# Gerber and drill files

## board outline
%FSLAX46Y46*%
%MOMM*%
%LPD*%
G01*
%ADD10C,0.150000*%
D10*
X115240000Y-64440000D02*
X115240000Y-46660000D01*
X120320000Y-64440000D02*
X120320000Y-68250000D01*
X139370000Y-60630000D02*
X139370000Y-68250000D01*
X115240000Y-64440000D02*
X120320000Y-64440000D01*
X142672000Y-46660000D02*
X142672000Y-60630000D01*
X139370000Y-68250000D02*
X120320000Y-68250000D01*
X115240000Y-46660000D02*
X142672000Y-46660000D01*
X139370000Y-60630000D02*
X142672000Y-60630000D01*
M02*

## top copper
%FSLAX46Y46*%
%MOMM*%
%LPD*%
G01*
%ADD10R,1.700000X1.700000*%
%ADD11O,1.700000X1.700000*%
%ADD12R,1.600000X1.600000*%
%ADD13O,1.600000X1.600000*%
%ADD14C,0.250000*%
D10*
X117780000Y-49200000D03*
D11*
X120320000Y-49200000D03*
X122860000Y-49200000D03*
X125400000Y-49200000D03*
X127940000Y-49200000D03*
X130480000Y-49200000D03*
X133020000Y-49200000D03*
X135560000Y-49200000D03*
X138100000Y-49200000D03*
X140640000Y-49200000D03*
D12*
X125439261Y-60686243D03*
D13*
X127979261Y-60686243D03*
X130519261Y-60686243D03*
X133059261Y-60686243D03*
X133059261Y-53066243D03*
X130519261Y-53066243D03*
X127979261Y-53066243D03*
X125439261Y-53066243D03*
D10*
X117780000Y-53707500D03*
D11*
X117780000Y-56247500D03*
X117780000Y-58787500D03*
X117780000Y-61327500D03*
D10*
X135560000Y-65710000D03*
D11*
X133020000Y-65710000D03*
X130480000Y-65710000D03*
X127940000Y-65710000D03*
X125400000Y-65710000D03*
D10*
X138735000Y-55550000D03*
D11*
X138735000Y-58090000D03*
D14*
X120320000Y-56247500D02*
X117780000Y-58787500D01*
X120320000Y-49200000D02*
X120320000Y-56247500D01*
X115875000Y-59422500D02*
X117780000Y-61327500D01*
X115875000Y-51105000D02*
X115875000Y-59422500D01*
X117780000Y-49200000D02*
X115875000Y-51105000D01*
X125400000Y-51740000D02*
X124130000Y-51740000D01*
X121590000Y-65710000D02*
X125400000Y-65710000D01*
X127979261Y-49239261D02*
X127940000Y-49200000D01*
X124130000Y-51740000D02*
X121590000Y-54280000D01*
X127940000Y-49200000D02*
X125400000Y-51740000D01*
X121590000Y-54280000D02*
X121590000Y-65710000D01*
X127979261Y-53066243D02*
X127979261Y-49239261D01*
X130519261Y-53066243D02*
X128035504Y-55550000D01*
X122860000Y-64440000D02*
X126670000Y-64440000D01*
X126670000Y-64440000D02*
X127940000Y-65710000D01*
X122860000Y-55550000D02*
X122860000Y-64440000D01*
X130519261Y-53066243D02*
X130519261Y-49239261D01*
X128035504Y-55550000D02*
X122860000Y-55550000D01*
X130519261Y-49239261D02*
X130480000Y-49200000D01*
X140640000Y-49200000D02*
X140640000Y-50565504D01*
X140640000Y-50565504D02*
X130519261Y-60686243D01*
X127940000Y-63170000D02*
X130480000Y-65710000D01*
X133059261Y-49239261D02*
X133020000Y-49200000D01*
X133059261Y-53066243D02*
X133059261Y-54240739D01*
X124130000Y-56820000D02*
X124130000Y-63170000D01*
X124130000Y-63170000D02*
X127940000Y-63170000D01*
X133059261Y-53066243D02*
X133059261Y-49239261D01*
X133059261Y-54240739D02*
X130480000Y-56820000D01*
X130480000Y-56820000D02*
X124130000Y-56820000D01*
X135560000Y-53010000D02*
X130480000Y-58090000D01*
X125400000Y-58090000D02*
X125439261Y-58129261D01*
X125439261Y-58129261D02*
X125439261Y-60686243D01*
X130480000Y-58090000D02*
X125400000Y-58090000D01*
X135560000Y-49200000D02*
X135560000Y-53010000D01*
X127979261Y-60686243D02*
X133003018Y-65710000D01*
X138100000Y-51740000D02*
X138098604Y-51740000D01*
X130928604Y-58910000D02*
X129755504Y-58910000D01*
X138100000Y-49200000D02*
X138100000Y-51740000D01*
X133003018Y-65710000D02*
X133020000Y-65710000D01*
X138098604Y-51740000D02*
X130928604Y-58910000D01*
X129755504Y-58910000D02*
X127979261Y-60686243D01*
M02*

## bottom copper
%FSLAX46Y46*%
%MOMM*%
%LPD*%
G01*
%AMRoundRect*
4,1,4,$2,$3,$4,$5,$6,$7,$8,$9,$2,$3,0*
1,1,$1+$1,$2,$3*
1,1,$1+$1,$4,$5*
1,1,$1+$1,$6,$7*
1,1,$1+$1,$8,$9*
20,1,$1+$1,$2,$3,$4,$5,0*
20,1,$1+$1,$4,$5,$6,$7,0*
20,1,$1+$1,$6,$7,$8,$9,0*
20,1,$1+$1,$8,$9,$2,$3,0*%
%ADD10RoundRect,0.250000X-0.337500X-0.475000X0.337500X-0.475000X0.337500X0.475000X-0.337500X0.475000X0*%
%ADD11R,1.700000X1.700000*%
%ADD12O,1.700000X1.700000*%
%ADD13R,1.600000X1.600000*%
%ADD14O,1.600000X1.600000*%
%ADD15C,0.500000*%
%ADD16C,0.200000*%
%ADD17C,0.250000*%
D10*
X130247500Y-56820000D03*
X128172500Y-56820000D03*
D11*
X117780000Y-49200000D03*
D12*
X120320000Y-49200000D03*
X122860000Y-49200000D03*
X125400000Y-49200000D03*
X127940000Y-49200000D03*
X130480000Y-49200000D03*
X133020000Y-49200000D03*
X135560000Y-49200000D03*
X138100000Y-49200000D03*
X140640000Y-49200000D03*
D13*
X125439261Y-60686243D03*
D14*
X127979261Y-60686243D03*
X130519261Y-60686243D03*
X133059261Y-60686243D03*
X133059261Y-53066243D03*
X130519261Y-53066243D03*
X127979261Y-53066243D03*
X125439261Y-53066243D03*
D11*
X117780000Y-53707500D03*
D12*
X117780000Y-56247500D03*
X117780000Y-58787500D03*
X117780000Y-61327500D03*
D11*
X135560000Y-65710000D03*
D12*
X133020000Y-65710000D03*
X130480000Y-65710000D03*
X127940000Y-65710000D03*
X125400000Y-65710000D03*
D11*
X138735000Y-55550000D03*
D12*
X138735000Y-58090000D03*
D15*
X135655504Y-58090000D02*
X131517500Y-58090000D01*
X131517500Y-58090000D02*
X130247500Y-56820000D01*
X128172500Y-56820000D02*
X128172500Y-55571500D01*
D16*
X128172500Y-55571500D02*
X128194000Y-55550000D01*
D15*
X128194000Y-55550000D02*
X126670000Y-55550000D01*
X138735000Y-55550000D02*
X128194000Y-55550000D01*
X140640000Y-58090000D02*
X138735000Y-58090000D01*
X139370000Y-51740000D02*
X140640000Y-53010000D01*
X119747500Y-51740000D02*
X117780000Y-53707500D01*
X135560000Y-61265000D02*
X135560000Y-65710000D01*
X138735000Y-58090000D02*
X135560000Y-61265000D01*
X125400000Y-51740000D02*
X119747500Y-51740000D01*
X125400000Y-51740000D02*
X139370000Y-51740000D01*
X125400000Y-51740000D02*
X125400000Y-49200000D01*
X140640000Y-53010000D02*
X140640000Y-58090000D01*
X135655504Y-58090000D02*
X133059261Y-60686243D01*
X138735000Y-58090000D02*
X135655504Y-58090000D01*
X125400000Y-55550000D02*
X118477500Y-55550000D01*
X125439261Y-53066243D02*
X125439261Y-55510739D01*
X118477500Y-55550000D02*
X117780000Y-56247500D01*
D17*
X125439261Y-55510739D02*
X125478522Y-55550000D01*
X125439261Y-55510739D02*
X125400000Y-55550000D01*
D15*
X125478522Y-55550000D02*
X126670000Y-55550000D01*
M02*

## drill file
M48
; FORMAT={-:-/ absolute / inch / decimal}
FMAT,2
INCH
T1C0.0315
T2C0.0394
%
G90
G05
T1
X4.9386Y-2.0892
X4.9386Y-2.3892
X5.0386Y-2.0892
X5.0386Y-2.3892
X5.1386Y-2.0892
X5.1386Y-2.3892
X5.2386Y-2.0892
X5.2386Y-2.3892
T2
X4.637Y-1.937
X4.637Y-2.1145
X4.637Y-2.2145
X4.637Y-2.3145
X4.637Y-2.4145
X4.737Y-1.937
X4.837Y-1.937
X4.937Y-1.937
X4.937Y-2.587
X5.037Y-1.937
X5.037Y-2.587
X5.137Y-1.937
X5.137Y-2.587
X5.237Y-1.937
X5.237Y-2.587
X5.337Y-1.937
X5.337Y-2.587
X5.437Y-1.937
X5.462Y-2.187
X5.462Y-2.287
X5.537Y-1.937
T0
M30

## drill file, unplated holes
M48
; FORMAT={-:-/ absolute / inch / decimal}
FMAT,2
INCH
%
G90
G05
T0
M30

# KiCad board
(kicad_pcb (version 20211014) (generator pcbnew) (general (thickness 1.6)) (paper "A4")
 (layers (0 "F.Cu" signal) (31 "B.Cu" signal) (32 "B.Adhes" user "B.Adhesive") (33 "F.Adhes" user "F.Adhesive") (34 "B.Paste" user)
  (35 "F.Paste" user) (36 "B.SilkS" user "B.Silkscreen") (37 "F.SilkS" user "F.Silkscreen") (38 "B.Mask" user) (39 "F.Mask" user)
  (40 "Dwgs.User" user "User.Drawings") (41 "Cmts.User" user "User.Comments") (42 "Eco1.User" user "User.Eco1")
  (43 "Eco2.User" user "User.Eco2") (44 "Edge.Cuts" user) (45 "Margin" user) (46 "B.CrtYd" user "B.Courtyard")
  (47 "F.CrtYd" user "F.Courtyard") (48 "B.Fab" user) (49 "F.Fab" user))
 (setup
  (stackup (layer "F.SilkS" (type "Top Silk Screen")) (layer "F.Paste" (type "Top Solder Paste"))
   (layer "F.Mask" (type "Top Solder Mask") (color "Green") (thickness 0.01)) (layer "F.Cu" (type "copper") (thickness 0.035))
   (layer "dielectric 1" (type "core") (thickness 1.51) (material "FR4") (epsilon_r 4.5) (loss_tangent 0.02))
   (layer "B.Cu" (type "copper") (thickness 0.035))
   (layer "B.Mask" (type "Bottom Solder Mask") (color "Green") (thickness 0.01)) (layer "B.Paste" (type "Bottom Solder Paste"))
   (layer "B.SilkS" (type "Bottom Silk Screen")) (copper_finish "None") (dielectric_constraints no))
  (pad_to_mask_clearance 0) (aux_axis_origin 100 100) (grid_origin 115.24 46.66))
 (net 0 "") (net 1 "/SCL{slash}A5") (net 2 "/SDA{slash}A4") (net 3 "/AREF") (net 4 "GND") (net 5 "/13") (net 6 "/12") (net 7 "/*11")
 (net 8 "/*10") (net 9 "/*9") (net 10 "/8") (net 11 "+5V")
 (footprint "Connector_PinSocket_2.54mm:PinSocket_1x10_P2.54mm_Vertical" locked (layer "F.Cu") (at 117.78 49.2 90)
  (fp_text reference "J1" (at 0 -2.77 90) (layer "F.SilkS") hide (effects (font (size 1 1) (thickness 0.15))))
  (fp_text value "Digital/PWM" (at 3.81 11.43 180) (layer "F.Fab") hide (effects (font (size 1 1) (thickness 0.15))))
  (pad "1" thru_hole rect locked (at 0 0 90) (size 1.7 1.7) (drill 1) (layers *.Cu *.Mask) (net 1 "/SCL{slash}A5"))
  (pad "2" thru_hole oval locked (at 0 2.54 90) (size 1.7 1.7) (drill 1) (layers *.Cu *.Mask) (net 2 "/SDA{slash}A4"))
  (pad "3" thru_hole oval locked (at 0 5.08 90) (size 1.7 1.7) (drill 1) (layers *.Cu *.Mask) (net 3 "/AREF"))
  (pad "4" thru_hole oval locked (at 0 7.62 90) (size 1.7 1.7) (drill 1) (layers *.Cu *.Mask) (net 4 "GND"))
  (pad "5" thru_hole oval locked (at 0 10.16 90) (size 1.7 1.7) (drill 1) (layers *.Cu *.Mask) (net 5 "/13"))
  (pad "6" thru_hole oval locked (at 0 12.7 90) (size 1.7 1.7) (drill 1) (layers *.Cu *.Mask) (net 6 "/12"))
  (pad "7" thru_hole oval locked (at 0 15.24 90) (size 1.7 1.7) (drill 1) (layers *.Cu *.Mask) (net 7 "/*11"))
  (pad "8" thru_hole oval locked (at 0 17.78 90) (size 1.7 1.7) (drill 1) (layers *.Cu *.Mask) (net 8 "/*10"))
  (pad "9" thru_hole oval locked (at 0 20.32 90) (size 1.7 1.7) (drill 1) (layers *.Cu *.Mask) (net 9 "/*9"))
  (pad "10" thru_hole oval locked (at 0 22.86 90) (size 1.7 1.7) (drill 1) (layers *.Cu *.Mask) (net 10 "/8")))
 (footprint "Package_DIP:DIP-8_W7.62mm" (layer "F.Cu") (at 125.439261 60.686243 90)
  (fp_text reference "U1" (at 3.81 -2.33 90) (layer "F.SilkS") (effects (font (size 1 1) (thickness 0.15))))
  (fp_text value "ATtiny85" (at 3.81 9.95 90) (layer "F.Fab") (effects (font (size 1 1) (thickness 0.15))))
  (pad "1" thru_hole rect (at 0 0 90) (size 1.6 1.6) (drill 0.8) (layers *.Cu *.Mask) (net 8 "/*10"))
  (pad "2" thru_hole oval (at 0 2.54 90) (size 1.6 1.6) (drill 0.8) (layers *.Cu *.Mask) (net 9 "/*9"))
  (pad "3" thru_hole oval (at 0 5.08 90) (size 1.6 1.6) (drill 0.8) (layers *.Cu *.Mask) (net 10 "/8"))
  (pad "4" thru_hole oval (at 0 7.62 90) (size 1.6 1.6) (drill 0.8) (layers *.Cu *.Mask) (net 4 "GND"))
  (pad "5" thru_hole oval (at 7.62 7.62 90) (size 1.6 1.6) (drill 0.8) (layers *.Cu *.Mask) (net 7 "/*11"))
  (pad "6" thru_hole oval (at 7.62 5.08 90) (size 1.6 1.6) (drill 0.8) (layers *.Cu *.Mask) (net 6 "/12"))
  (pad "7" thru_hole oval (at 7.62 2.54 90) (size 1.6 1.6) (drill 0.8) (layers *.Cu *.Mask) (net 5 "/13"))
  (pad "8" thru_hole oval (at 7.62 0 90) (size 1.6 1.6) (drill 0.8) (layers *.Cu *.Mask) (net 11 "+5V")))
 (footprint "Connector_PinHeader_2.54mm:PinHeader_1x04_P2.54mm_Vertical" (layer "F.Cu") (at 117.78 53.7075)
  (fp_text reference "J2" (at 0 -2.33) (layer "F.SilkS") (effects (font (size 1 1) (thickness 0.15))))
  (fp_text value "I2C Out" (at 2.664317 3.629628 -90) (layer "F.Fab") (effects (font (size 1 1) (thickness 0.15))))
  (pad "1" thru_hole rect (at 0 0) (size 1.7 1.7) (drill 1) (layers *.Cu *.Mask) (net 4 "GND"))
  (pad "2" thru_hole oval (at 0 2.54) (size 1.7 1.7) (drill 1) (layers *.Cu *.Mask) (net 11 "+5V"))
  (pad "3" thru_hole oval (at 0 5.08) (size 1.7 1.7) (drill 1) (layers *.Cu *.Mask) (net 2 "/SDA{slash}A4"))
  (pad "4" thru_hole oval (at 0 7.62) (size 1.7 1.7) (drill 1) (layers *.Cu *.Mask) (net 1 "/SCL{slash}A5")))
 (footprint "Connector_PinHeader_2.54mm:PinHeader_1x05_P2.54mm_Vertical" (layer "F.Cu") (at 135.56 65.71 -90)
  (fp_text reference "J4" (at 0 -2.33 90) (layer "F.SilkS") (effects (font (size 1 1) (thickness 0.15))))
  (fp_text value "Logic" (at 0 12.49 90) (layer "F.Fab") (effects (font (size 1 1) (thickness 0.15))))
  (pad "1" thru_hole rect (at 0 0 270) (size 1.7 1.7) (drill 1) (layers *.Cu *.Mask) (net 4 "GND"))
  (pad "2" thru_hole oval (at 0 2.54 270) (size 1.7 1.7) (drill 1) (layers *.Cu *.Mask) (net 9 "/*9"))
  (pad "3" thru_hole oval (at 0 5.08 270) (size 1.7 1.7) (drill 1) (layers *.Cu *.Mask) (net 7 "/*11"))
  (pad "4" thru_hole oval (at 0 7.62 270) (size 1.7 1.7) (drill 1) (layers *.Cu *.Mask) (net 6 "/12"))
  (pad "5" thru_hole oval (at 0 10.16 270) (size 1.7 1.7) (drill 1) (layers *.Cu *.Mask) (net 5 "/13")))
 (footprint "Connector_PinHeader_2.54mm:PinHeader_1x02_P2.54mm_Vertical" (layer "F.Cu") (at 138.735 55.55)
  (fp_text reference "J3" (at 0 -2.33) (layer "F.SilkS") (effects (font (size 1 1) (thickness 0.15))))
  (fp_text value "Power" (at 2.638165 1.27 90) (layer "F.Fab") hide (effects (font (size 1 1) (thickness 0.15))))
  (pad "1" thru_hole rect (at 0 0) (size 1.7 1.7) (drill 1) (layers *.Cu *.Mask) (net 11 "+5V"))
  (pad "2" thru_hole oval (at 0 2.54) (size 1.7 1.7) (drill 1) (layers *.Cu *.Mask) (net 4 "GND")))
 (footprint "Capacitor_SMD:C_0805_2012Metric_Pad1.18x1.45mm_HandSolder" (layer "B.Cu") (at 129.21 56.82)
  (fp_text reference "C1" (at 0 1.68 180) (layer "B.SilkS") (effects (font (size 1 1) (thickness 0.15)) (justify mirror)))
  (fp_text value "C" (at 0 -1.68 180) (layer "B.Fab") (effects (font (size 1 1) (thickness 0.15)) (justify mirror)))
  (pad "1" smd roundrect (at -1.0375 0) (size 1.175 1.45) (layers "B.Cu" "B.Paste" "B.Mask") (roundrect_rratio 0.212766) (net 11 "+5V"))
  (pad "2" smd roundrect (at 1.0375 0) (size 1.175 1.45) (layers "B.Cu" "B.Paste" "B.Mask") (roundrect_rratio 0.212766) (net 4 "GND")))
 (gr_line (start 115.24 64.44) (end 115.24 46.66) (layer "Edge.Cuts") (width 0.15))
 (gr_line (start 120.32 64.44) (end 120.32 68.25) (layer "Edge.Cuts") (width 0.15))
 (gr_line (start 139.37 60.63) (end 139.37 68.25) (layer "Edge.Cuts") (width 0.15))
 (gr_line (start 115.24 64.44) (end 120.32 64.44) (layer "Edge.Cuts") (width 0.15))
 (gr_line (start 142.672 46.66) (end 142.672 60.63) (layer "Edge.Cuts") (width 0.15))
 (gr_line (start 139.37 68.25) (end 120.32 68.25) (layer "Edge.Cuts") (width 0.15))
 (gr_line (start 115.24 46.66) (end 142.672 46.66) (layer "Edge.Cuts") (width 0.15))
 (gr_line (start 139.37 60.63) (end 142.672 60.63) (layer "Edge.Cuts") (width 0.15))
 (segment (start 131.5175 58.09) (end 130.2475 56.82) (width 0.5) (layer "B.Cu") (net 4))
 (segment (start 140.64 58.09) (end 138.735 58.09) (width 0.5) (layer "B.Cu") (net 4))
 (segment (start 139.37 51.74) (end 140.64 53.01) (width 0.5) (layer "B.Cu") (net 4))
 (segment (start 119.7475 51.74) (end 117.78 53.7075) (width 0.5) (layer "B.Cu") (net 4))
 (segment (start 135.56 61.265) (end 135.56 65.71) (width 0.5) (layer "B.Cu") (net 4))
 (segment (start 138.735 58.09) (end 135.56 61.265) (width 0.5) (layer "B.Cu") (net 4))
 (segment (start 135.655504 58.09) (end 131.5175 58.09) (width 0.5) (layer "B.Cu") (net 4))
 (segment (start 125.4 51.74) (end 119.7475 51.74) (width 0.5) (layer "B.Cu") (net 4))
 (segment (start 125.4 51.74) (end 139.37 51.74) (width 0.5) (layer "B.Cu") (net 4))
 (segment (start 125.4 51.74) (end 125.4 49.2) (width 0.5) (layer "B.Cu") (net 4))
 (segment (start 140.64 53.01) (end 140.64 58.09) (width 0.5) (layer "B.Cu") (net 4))
 (segment (start 135.655504 58.09) (end 133.059261 60.686243) (width 0.5) (layer "B.Cu") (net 4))
 (segment (start 138.735 58.09) (end 135.655504 58.09) (width 0.5) (layer "B.Cu") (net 4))
 (segment (start 125.4 55.55) (end 118.4775 55.55) (width 0.5) (layer "B.Cu") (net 11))
 (segment (start 128.1725 56.82) (end 128.1725 55.5715) (width 0.5) (layer "B.Cu") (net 11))
 (segment (start 128.194 55.55) (end 126.67 55.55) (width 0.5) (layer "B.Cu") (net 11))
 (segment (start 125.439261 53.066243) (end 125.439261 55.510739) (width 0.5) (layer "B.Cu") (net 11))
 (segment (start 128.1725 55.5715) (end 128.194 55.55) (width 0.2) (layer "B.Cu") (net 11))
 (segment (start 118.4775 55.55) (end 117.78 56.2475) (width 0.5) (layer "B.Cu") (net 11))
 (segment (start 138.735 55.55) (end 128.194 55.55) (width 0.5) (layer "B.Cu") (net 11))
 (segment (start 125.439261 55.510739) (end 125.478522 55.55) (width 0.25) (layer "B.Cu") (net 11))
 (segment (start 125.439261 55.510739) (end 125.4 55.55) (width 0.25) (layer "B.Cu") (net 11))
 (segment (start 125.478522 55.55) (end 126.67 55.55) (width 0.5) (layer "B.Cu") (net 11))
 (segment (start 120.32 56.2475) (end 117.78 58.7875) (width 0.25) (layer "F.Cu") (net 2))
 (segment (start 120.32 49.2) (end 120.32 56.2475) (width 0.25) (layer "F.Cu") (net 2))
 (segment (start 115.875 51.105) (end 115.875 59.4225) (width 0.25) (layer "F.Cu") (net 1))
 (segment (start 117.78 49.2) (end 115.875 51.105) (width 0.25) (layer "F.Cu") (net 1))
 (segment (start 115.875 59.4225) (end 117.78 61.3275) (width 0.25) (layer "F.Cu") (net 1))
 (segment (start 125.4 51.74) (end 124.13 51.74) (width 0.25) (layer "F.Cu") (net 5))
 (segment (start 121.59 65.71) (end 125.4 65.71) (width 0.25) (layer "F.Cu") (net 5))
 (segment (start 127.979261 49.239261) (end 127.94 49.2) (width 0.25) (layer "F.Cu") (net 5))
 (segment (start 124.13 51.74) (end 121.59 54.28) (width 0.25) (layer "F.Cu") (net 5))
 (segment (start 127.94 49.2) (end 125.4 51.74) (width 0.25) (layer "F.Cu") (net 5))
 (segment (start 121.59 54.28) (end 121.59 65.71) (width 0.25) (layer "F.Cu") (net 5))
 (segment (start 127.979261 53.066243) (end 127.979261 49.239261) (width 0.25) (layer "F.Cu") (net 5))
 (segment (start 130.519261 53.066243) (end 128.035504 55.55) (width 0.25) (layer "F.Cu") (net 6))
 (segment (start 122.86 64.44) (end 126.67 64.44) (width 0.25) (layer "F.Cu") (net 6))
 (segment (start 126.67 64.44) (end 127.94 65.71) (width 0.25) (layer "F.Cu") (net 6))
 (segment (start 122.86 55.55) (end 122.86 64.44) (width 0.25) (layer "F.Cu") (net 6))
 (segment (start 130.519261 53.066243) (end 130.519261 49.239261) (width 0.25) (layer "F.Cu") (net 6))
 (segment (start 128.035504 55.55) (end 122.86 55.55) (width 0.25) (layer "F.Cu") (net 6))
 (segment (start 130.519261 49.239261) (end 130.48 49.2) (width 0.25) (layer "F.Cu") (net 6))
 (segment (start 140.64 49.2) (end 140.64 50.565504) (width 0.25) (layer "F.Cu") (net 10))
 (segment (start 140.64 50.565504) (end 130.519261 60.686243) (width 0.25) (layer "F.Cu") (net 10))
 (segment (start 127.94 63.17) (end 130.48 65.71) (width 0.25) (layer "F.Cu") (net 7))
 (segment (start 133.059261 49.239261) (end 133.02 49.2) (width 0.25) (layer "F.Cu") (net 7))
 (segment (start 133.059261 53.066243) (end 133.059261 54.240739) (width 0.25) (layer "F.Cu") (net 7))
 (segment (start 124.13 56.82) (end 124.13 63.17) (width 0.25) (layer "F.Cu") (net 7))
 (segment (start 124.13 63.17) (end 127.94 63.17) (width 0.25) (layer "F.Cu") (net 7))
 (segment (start 133.059261 53.066243) (end 133.059261 49.239261) (width 0.25) (layer "F.Cu") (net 7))
 (segment (start 133.059261 54.240739) (end 130.48 56.82) (width 0.25) (layer "F.Cu") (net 7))
 (segment (start 130.48 56.82) (end 124.13 56.82) (width 0.25) (layer "F.Cu") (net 7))
 (segment (start 135.56 53.01) (end 130.48 58.09) (width 0.25) (layer "F.Cu") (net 8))
 (segment (start 125.4 58.09) (end 125.439261 58.129261) (width 0.25) (layer "F.Cu") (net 8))
 (segment (start 125.439261 58.129261) (end 125.439261 60.686243) (width 0.25) (layer "F.Cu") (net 8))
 (segment (start 130.48 58.09) (end 125.4 58.09) (width 0.25) (layer "F.Cu") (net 8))
 (segment (start 135.56 49.2) (end 135.56 53.01) (width 0.25) (layer "F.Cu") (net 8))
 (segment (start 127.979261 60.686243) (end 133.003018 65.71) (width 0.25) (layer "F.Cu") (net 9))
 (segment (start 138.1 51.74) (end 138.098604 51.74) (width 0.25) (layer "F.Cu") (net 9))
 (segment (start 130.928604 58.91) (end 129.755504 58.91) (width 0.25) (layer "F.Cu") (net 9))
 (segment (start 138.1 49.2) (end 138.1 51.74) (width 0.25) (layer "F.Cu") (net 9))
 (segment (start 133.003018 65.71) (end 133.02 65.71) (width 0.25) (layer "F.Cu") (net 9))
 (segment (start 138.098604 51.74) (end 130.928604 58.91) (width 0.25) (layer "F.Cu") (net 9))
 (segment (start 129.755504 58.91) (end 127.979261 60.686243) (width 0.25) (layer "F.Cu") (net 9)))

